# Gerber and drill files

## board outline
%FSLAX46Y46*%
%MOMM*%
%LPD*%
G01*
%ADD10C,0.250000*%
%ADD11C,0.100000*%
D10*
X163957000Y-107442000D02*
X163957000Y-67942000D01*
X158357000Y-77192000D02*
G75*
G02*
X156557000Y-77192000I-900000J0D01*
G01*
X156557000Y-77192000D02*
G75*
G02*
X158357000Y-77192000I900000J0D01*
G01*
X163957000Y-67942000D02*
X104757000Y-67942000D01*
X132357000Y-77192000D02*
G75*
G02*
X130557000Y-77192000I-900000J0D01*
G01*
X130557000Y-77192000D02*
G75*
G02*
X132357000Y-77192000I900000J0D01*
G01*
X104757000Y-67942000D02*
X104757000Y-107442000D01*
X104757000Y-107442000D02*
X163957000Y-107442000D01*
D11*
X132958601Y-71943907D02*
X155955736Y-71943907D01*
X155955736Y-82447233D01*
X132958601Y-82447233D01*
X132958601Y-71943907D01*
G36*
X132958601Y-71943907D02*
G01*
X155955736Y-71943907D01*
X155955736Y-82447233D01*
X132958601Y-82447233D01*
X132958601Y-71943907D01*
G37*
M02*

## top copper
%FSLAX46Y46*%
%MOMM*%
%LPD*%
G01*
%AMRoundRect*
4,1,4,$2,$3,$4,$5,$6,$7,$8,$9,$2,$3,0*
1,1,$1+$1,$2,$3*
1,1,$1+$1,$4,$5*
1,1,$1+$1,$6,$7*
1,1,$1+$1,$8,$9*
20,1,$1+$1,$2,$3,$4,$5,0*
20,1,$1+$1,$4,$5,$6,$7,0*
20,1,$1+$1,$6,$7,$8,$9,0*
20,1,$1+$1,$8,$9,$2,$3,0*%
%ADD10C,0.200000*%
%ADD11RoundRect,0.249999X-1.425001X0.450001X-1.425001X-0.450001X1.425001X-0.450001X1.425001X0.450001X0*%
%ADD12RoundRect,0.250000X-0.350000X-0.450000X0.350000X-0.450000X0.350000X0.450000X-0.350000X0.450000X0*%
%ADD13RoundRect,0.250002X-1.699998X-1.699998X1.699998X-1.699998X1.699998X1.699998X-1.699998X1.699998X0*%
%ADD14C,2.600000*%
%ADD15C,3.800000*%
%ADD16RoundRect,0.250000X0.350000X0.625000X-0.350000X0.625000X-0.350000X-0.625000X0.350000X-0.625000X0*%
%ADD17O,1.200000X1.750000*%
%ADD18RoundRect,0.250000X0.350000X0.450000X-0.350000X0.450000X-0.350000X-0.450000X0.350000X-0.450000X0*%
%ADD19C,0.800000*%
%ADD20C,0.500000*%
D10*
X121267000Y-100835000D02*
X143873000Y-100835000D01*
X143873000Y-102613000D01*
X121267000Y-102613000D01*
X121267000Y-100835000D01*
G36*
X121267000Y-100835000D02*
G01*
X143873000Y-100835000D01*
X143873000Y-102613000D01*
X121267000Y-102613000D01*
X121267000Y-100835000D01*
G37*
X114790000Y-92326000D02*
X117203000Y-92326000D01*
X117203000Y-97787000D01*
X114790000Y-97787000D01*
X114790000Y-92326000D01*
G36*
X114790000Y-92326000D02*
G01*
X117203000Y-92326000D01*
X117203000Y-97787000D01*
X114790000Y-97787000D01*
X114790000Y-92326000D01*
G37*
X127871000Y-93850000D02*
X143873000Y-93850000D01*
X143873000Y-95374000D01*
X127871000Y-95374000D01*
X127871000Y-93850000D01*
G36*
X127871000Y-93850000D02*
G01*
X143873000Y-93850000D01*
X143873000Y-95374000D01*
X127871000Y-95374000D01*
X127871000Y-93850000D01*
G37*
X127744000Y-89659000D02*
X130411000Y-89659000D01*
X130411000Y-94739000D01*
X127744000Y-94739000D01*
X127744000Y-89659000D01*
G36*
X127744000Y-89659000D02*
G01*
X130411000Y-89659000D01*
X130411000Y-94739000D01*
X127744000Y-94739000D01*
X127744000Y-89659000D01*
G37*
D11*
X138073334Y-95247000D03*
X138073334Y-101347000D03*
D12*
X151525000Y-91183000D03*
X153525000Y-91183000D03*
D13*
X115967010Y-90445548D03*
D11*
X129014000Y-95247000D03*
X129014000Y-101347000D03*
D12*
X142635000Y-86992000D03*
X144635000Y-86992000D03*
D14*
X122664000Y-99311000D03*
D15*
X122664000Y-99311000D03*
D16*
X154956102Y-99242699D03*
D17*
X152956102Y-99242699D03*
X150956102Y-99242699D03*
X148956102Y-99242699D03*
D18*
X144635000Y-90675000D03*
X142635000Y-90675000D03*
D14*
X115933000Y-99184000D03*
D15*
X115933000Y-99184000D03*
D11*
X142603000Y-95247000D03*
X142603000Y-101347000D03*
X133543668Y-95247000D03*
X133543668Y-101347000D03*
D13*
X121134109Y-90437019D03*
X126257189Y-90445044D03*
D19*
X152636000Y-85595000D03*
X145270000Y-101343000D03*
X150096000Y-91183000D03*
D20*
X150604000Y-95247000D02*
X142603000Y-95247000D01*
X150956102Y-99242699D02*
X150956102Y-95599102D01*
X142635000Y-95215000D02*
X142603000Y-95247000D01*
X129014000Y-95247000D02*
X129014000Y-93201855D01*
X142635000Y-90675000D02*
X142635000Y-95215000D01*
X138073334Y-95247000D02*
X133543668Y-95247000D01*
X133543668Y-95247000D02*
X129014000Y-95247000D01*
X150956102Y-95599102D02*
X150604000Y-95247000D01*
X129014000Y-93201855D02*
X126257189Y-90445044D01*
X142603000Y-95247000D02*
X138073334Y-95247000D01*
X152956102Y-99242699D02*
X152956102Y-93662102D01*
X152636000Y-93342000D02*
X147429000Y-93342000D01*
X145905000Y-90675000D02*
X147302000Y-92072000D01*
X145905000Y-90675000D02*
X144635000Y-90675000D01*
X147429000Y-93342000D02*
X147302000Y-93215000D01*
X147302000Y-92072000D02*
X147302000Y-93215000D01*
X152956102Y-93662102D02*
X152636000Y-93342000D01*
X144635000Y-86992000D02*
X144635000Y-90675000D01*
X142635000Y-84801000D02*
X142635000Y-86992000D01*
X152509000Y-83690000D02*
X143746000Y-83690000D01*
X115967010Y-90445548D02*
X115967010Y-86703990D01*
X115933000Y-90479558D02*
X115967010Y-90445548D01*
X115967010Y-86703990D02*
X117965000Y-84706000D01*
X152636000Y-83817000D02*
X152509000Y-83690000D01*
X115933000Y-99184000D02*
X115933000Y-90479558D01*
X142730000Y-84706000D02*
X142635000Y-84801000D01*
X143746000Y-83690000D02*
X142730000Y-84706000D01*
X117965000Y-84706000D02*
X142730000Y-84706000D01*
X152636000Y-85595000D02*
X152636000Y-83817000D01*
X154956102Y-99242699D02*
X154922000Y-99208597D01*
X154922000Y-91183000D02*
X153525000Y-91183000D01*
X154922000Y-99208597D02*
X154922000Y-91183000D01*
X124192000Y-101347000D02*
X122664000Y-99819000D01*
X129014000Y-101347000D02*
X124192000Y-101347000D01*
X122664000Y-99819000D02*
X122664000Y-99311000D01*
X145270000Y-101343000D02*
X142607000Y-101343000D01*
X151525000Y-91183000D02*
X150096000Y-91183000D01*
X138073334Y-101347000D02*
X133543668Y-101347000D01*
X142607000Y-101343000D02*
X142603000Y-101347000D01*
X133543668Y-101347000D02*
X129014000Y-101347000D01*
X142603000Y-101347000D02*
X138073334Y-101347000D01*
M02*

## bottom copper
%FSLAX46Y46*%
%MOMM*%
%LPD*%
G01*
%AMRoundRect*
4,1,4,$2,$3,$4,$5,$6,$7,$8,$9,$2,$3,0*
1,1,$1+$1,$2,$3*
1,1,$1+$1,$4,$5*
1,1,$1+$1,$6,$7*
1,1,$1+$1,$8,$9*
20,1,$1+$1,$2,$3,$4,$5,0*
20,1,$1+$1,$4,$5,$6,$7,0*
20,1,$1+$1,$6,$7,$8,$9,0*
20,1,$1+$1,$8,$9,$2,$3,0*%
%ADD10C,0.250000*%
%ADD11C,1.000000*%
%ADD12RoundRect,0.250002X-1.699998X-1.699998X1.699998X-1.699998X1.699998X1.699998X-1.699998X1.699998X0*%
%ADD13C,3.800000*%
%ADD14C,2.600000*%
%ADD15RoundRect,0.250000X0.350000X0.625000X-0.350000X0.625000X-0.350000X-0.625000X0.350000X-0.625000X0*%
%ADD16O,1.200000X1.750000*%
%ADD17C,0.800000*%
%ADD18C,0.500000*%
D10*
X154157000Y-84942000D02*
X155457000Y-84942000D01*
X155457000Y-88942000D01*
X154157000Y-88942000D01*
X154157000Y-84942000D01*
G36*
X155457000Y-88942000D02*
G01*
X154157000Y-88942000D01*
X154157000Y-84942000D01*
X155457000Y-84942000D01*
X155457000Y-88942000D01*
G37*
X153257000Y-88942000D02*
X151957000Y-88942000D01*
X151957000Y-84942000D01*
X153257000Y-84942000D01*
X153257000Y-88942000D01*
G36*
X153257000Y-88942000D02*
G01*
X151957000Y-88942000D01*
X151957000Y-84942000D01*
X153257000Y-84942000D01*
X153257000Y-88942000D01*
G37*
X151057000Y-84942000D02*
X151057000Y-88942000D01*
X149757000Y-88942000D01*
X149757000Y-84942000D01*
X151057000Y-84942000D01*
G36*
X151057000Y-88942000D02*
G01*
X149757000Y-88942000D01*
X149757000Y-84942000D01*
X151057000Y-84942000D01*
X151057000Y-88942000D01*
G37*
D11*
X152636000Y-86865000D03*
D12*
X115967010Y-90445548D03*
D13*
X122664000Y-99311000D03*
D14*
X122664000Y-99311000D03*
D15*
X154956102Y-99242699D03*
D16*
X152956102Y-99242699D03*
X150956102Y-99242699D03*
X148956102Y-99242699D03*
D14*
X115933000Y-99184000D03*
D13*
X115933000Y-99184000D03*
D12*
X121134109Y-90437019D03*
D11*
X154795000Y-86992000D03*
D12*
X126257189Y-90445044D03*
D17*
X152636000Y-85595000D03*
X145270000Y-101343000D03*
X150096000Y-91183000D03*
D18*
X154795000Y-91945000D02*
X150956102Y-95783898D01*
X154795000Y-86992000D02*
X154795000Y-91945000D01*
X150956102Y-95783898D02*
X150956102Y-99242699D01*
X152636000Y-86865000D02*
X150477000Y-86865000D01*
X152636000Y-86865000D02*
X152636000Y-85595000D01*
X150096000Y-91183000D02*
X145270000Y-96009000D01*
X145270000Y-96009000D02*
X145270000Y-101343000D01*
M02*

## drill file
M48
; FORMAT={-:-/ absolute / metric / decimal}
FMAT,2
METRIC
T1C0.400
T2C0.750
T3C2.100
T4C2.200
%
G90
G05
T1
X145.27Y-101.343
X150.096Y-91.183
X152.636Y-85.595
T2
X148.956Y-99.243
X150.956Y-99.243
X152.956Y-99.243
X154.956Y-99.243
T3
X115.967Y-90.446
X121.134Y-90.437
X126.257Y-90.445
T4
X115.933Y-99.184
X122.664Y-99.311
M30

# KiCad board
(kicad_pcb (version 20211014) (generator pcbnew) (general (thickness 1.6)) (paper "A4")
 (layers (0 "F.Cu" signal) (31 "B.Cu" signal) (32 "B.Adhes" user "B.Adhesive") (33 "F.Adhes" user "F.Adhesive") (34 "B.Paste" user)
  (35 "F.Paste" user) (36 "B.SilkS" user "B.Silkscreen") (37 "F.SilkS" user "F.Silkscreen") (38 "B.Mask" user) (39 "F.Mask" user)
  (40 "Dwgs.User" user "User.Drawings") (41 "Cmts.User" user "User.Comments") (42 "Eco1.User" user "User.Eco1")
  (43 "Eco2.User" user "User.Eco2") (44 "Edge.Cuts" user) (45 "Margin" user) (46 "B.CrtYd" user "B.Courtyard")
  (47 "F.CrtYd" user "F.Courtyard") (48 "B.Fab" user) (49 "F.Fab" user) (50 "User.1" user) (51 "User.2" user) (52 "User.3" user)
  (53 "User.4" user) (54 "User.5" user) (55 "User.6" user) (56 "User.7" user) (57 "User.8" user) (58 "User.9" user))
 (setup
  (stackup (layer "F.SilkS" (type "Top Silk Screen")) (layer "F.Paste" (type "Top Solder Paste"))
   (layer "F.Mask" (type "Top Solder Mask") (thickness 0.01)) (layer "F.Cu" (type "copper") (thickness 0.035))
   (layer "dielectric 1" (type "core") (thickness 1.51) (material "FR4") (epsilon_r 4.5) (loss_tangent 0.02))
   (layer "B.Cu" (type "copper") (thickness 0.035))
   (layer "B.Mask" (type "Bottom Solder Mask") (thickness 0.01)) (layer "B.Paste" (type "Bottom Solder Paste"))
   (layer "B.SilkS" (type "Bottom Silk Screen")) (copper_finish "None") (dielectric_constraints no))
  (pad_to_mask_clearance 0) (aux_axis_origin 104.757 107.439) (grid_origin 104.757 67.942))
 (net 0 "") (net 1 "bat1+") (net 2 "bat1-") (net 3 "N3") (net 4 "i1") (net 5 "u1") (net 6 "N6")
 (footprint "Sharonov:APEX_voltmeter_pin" (layer "F.Cu") (at 152.636 86.865)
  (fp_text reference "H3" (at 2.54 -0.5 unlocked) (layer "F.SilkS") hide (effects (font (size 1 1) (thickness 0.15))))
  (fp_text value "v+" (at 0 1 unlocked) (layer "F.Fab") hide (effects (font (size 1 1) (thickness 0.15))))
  (pad "1" smd circle (at 0 0) (size 1 1) (layers "B.Cu") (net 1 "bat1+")))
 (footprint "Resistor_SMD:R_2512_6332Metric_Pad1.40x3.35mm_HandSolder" (layer "F.Cu") (at 138.073334 98.297 -90)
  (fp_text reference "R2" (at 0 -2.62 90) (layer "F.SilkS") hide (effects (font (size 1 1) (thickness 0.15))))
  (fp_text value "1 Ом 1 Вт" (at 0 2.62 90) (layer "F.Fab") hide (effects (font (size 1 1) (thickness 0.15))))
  (pad "1" smd roundrect locked (at -3.05 0 270) (size 1.4 3.35) (layers "F.Cu" "F.Paste" "F.Mask") (roundrect_rratio 0.1785707143)
   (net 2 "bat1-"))
  (pad "2" smd roundrect locked (at 3.05 0 270) (size 1.4 3.35) (layers "F.Cu" "F.Paste" "F.Mask") (roundrect_rratio 0.1785707143)
   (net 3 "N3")))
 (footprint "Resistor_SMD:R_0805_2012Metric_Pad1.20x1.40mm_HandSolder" (layer "F.Cu") (at 152.525 91.183)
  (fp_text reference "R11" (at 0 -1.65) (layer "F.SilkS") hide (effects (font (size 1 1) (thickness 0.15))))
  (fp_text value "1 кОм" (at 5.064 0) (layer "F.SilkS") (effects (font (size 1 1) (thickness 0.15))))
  (pad "1" smd roundrect locked (at -1 0) (size 1.2 1.4) (layers "F.Cu" "F.Paste" "F.Mask") (roundrect_rratio 0.2083333333) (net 3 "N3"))
  (pad "2" smd roundrect locked (at 1 0) (size 1.2 1.4) (layers "F.Cu" "F.Paste" "F.Mask") (roundrect_rratio 0.2083333333) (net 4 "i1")))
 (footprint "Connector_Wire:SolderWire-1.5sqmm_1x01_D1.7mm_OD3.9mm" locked (layer "F.Cu") (at 115.96701 90.445548)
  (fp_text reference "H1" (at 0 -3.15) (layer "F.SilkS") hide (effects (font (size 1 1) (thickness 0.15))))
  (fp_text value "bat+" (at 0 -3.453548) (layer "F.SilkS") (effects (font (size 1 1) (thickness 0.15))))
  (pad "1" thru_hole roundrect locked (at 0 0) (size 3.9 3.9) (drill 2.1) (layers *.Cu *.Mask) (roundrect_rratio 0.06410307692)
   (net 1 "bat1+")))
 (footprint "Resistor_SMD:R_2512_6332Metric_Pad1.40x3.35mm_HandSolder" (layer "F.Cu") (at 129.014 98.297 -90)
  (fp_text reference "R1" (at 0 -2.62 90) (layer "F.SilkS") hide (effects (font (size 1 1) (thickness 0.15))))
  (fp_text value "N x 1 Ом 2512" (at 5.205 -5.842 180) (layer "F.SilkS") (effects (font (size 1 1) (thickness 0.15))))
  (pad "1" smd roundrect locked (at -3.05 0 270) (size 1.4 3.35) (layers "F.Cu" "F.Paste" "F.Mask") (roundrect_rratio 0.1785707143)
   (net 2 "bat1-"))
  (pad "2" smd roundrect locked (at 3.05 0 270) (size 1.4 3.35) (layers "F.Cu" "F.Paste" "F.Mask") (roundrect_rratio 0.1785707143)
   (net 3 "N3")))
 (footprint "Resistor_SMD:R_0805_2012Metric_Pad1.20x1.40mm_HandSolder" (layer "F.Cu") (at 143.635 86.992)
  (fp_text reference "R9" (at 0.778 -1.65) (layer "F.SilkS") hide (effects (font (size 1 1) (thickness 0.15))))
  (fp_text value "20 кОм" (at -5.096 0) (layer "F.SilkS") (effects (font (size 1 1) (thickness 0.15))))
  (pad "1" smd roundrect locked (at -1 0) (size 1.2 1.4) (layers "F.Cu" "F.Paste" "F.Mask") (roundrect_rratio 0.2083333333) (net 1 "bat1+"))
  (pad "2" smd roundrect locked (at 1 0) (size 1.2 1.4) (layers "F.Cu" "F.Paste" "F.Mask") (roundrect_rratio 0.2083333333) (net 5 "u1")))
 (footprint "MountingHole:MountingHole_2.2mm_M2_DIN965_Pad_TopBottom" (layer "F.Cu") (at 122.664 99.311)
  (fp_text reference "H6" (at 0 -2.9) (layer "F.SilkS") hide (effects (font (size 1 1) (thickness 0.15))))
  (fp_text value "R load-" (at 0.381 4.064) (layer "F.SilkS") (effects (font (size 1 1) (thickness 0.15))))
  (pad "1" connect circle locked (at 0 0) (size 3.8 3.8) (layers "B.Cu" "B.Mask") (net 3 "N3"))
  (pad "1" thru_hole circle locked (at 0 0) (size 2.6 2.6) (drill 2.2) (layers *.Cu *.Mask) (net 3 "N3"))
  (pad "1" connect circle locked (at 0 0) (size 3.8 3.8) (layers "F.Cu" "F.Mask") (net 3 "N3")))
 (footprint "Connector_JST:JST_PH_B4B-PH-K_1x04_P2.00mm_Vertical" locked (layer "F.Cu") (at 154.956102 99.242699 180)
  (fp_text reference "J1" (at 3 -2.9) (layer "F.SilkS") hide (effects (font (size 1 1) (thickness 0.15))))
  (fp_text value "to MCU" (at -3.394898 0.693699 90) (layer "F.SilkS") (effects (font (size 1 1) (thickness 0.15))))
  (pad "1" thru_hole roundrect locked (at 0 0 180) (size 1.2 1.75) (drill 0.75) (layers *.Cu *.Mask) (roundrect_rratio 0.2083333333)
   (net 4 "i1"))
  (pad "2" thru_hole oval locked (at 2 0 180) (size 1.2 1.75) (drill 0.75) (layers *.Cu *.Mask) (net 5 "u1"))
  (pad "3" thru_hole oval locked (at 4 0 180) (size 1.2 1.75) (drill 0.75) (layers *.Cu *.Mask) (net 2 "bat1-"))
  (pad "4" thru_hole oval locked (at 6 0 180) (size 1.2 1.75) (drill 0.75) (layers *.Cu *.Mask) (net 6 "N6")))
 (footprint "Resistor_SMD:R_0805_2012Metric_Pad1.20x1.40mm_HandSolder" (layer "F.Cu") (at 143.635 90.675 180)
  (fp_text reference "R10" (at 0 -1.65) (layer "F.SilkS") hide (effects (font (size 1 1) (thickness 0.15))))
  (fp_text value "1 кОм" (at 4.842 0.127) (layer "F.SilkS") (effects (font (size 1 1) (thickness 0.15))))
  (pad "1" smd roundrect locked (at -1 0 180) (size 1.2 1.4) (layers "F.Cu" "F.Paste" "F.Mask") (roundrect_rratio 0.2083333333) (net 5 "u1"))
  (pad "2" smd roundrect locked (at 1 0 180) (size 1.2 1.4) (layers "F.Cu" "F.Paste" "F.Mask") (roundrect_rratio 0.2083333333)
   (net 2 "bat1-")))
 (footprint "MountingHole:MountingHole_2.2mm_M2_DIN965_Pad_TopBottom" (layer "F.Cu") (at 115.933 99.184)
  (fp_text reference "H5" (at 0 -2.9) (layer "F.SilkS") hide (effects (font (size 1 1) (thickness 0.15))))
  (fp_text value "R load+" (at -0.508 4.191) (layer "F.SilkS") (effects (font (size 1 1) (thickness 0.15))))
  (pad "1" thru_hole circle locked (at 0 0) (size 2.6 2.6) (drill 2.2) (layers *.Cu *.Mask) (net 1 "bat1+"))
  (pad "1" connect circle locked (at 0 0) (size 3.8 3.8) (layers "F.Cu" "F.Mask") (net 1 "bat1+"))
  (pad "1" connect circle locked (at 0 0) (size 3.8 3.8) (layers "B.Cu" "B.Mask") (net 1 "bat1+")))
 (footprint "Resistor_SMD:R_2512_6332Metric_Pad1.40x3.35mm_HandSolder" (layer "F.Cu") (at 142.603 98.297 -90)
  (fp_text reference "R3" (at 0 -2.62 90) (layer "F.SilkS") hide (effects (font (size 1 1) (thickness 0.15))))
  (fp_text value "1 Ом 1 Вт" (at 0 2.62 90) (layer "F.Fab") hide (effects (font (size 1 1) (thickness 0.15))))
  (pad "1" smd roundrect locked (at -3.05 0 270) (size 1.4 3.35) (layers "F.Cu" "F.Paste" "F.Mask") (roundrect_rratio 0.1785707143)
   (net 2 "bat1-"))
  (pad "2" smd roundrect locked (at 3.05 0 270) (size 1.4 3.35) (layers "F.Cu" "F.Paste" "F.Mask") (roundrect_rratio 0.1785707143)
   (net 3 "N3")))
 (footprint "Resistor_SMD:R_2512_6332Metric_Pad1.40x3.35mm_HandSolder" (layer "F.Cu") (at 133.543668 98.297 -90)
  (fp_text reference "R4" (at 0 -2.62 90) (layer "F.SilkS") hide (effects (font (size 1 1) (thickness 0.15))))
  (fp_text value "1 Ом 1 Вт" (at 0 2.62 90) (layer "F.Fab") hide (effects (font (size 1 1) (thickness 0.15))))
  (pad "1" smd roundrect locked (at -3.05 0 270) (size 1.4 3.35) (layers "F.Cu" "F.Paste" "F.Mask") (roundrect_rratio 0.1785707143)
   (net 2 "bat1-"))
  (pad "2" smd roundrect locked (at 3.05 0 270) (size 1.4 3.35) (layers "F.Cu" "F.Paste" "F.Mask") (roundrect_rratio 0.1785707143)
   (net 3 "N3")))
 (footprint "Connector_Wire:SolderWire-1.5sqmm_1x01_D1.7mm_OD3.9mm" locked (layer "F.Cu") (at 121.134109 90.437019)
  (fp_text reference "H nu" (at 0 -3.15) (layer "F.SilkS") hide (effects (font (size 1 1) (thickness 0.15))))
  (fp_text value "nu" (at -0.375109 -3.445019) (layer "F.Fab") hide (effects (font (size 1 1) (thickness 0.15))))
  (pad "1" thru_hole roundrect locked (at 0 0) (size 3.9 3.9) (drill 2.1) (layers *.Cu *.Mask) (roundrect_rratio 0.06410307692)))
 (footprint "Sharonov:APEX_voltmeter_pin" (layer "F.Cu") (at 154.795 86.992)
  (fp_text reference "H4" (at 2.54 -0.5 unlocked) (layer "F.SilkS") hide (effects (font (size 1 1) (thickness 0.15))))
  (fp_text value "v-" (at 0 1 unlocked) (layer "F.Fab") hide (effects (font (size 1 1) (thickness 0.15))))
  (pad "1" smd circle (at 0 0) (size 1 1) (layers "B.Cu") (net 2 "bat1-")))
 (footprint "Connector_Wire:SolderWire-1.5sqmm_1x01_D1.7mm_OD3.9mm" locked (layer "F.Cu") (at 126.257189 90.445044)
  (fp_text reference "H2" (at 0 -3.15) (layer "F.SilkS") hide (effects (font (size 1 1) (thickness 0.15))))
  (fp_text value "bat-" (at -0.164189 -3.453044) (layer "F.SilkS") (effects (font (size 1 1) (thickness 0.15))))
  (pad "1" thru_hole roundrect locked (at 0 0) (size 3.9 3.9) (drill 2.1) (layers *.Cu *.Mask) (roundrect_rratio 0.06410307692)
   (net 2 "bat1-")))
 (gr_rect (start 143.873 102.613) (end 121.267 100.835) (layer "F.Cu") (width 0.2) (fill solid))
 (gr_rect (start 114.79 92.326) (end 117.203 97.787) (layer "F.Cu") (width 0.2) (fill solid))
 (gr_rect (start 127.871 95.374) (end 143.873 93.85) (layer "F.Cu") (width 0.2) (fill solid))
 (gr_rect (start 130.411 94.739) (end 127.744 89.659) (layer "F.Cu") (width 0.2) (fill solid))
 (gr_poly locked
  (pts (xy 154.157 84.942) (xy 155.457 84.942) (xy 155.457 88.942) (xy 154.157 88.942)) (layer "B.Cu") (width 0.25) (fill solid))
 (gr_poly locked
  (pts (xy 153.257 88.942) (xy 151.957 88.942) (xy 151.957 84.942) (xy 153.257 84.942)) (layer "B.Cu") (width 0.25) (fill solid))
 (gr_poly locked
  (pts (xy 151.057 84.942) (xy 151.057 88.942) (xy 149.757 88.942) (xy 149.757 84.942)) (layer "B.Cu") (width 0.25) (fill solid))
 (gr_line locked (start 163.957 107.442) (end 163.957 67.942) (layer "Edge.Cuts") (width 0.25))
 (gr_circle locked (center 157.457 77.192) (end 158.357 77.192) (layer "Edge.Cuts") (width 0.25) (fill none))
 (gr_line locked (start 163.957 67.942) (end 104.757 67.942) (layer "Edge.Cuts") (width 0.25))
 (gr_circle locked (center 131.457 77.192) (end 132.357 77.192) (layer "Edge.Cuts") (width 0.25) (fill none))
 (gr_line locked (start 104.757 67.942) (end 104.757 107.442) (layer "Edge.Cuts") (width 0.25))
 (gr_line locked (start 104.757 107.442) (end 163.957 107.442) (layer "Edge.Cuts") (width 0.25))
 (gr_rect locked (start 132.958601 71.943907) (end 155.955736 82.447233) (layer "Edge.Cuts") (width 0.1) (fill solid))
 (segment (start 150.604 95.247) (end 142.603 95.247) (width 0.5) (layer "F.Cu") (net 2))
 (segment (start 150.956102 99.242699) (end 150.956102 95.599102) (width 0.5) (layer "F.Cu") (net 2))
 (segment (start 142.635 95.215) (end 142.603 95.247) (width 0.5) (layer "F.Cu") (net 2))
 (segment (start 129.014 95.247) (end 129.014 93.201855) (width 0.5) (layer "F.Cu") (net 2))
 (segment (start 142.635 90.675) (end 142.635 95.215) (width 0.5) (layer "F.Cu") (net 2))
 (segment (start 138.073334 95.247) (end 133.543668 95.247) (width 0.5) (layer "F.Cu") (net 2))
 (segment (start 133.543668 95.247) (end 129.014 95.247) (width 0.5) (layer "F.Cu") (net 2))
 (segment (start 150.956102 95.599102) (end 150.604 95.247) (width 0.5) (layer "F.Cu") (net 2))
 (segment (start 129.014 93.201855) (end 126.257189 90.445044) (width 0.5) (layer "F.Cu") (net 2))
 (segment (start 142.603 95.247) (end 138.073334 95.247) (width 0.5) (layer "F.Cu") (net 2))
 (segment (start 154.795 91.945) (end 150.956102 95.783898) (width 0.5) (layer "B.Cu") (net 2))
 (segment (start 154.795 86.992) (end 154.795 91.945) (width 0.5) (layer "B.Cu") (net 2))
 (segment (start 150.956102 95.783898) (end 150.956102 99.242699) (width 0.5) (layer "B.Cu") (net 2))
 (segment (start 152.956102 99.242699) (end 152.956102 93.662102) (width 0.5) (layer "F.Cu") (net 5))
 (segment (start 152.636 93.342) (end 147.429 93.342) (width 0.5) (layer "F.Cu") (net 5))
 (segment (start 145.905 90.675) (end 147.302 92.072) (width 0.5) (layer "F.Cu") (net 5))
 (segment (start 145.905 90.675) (end 144.635 90.675) (width 0.5) (layer "F.Cu") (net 5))
 (segment (start 147.429 93.342) (end 147.302 93.215) (width 0.5) (layer "F.Cu") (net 5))
 (segment (start 147.302 92.072) (end 147.302 93.215) (width 0.5) (layer "F.Cu") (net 5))
 (segment (start 152.956102 93.662102) (end 152.636 93.342) (width 0.5) (layer "F.Cu") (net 5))
 (segment (start 144.635 86.992) (end 144.635 90.675) (width 0.5) (layer "F.Cu") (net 5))
 (segment (start 142.635 84.801) (end 142.635 86.992) (width 0.5) (layer "F.Cu") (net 1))
 (segment (start 152.509 83.69) (end 143.746 83.69) (width 0.5) (layer "F.Cu") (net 1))
 (segment (start 115.96701 90.445548) (end 115.96701 86.70399) (width 0.5) (layer "F.Cu") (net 1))
 (segment (start 115.933 90.479558) (end 115.96701 90.445548) (width 0.5) (layer "F.Cu") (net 1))
 (segment (start 115.96701 86.70399) (end 117.965 84.706) (width 0.5) (layer "F.Cu") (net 1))
 (segment (start 152.636 83.817) (end 152.509 83.69) (width 0.5) (layer "F.Cu") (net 1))
 (segment (start 115.933 99.184) (end 115.933 90.479558) (width 0.5) (layer "F.Cu") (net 1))
 (segment (start 142.73 84.706) (end 142.635 84.801) (width 0.5) (layer "F.Cu") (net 1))
 (segment (start 143.746 83.69) (end 142.73 84.706) (width 0.5) (layer "F.Cu") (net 1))
 (segment (start 117.965 84.706) (end 142.73 84.706) (width 0.5) (layer "F.Cu") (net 1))
 (segment (start 152.636 85.595) (end 152.636 83.817) (width 0.5) (layer "F.Cu") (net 1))
 (via (at 152.636 85.595) (size 0.8) (drill 0.4) (layers "F.Cu" "B.Cu") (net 1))
 (segment (start 152.636 86.865) (end 150.477 86.865) (width 0.5) (layer "B.Cu") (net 1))
 (segment (start 152.636 86.865) (end 152.636 85.595) (width 0.5) (layer "B.Cu") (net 1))
 (segment (start 154.956102 99.242699) (end 154.922 99.208597) (width 0.5) (layer "F.Cu") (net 4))
 (segment (start 154.922 91.183) (end 153.525 91.183) (width 0.5) (layer "F.Cu") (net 4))
 (segment (start 154.922 99.208597) (end 154.922 91.183) (width 0.5) (layer "F.Cu") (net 4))
 (segment (start 124.192 101.347) (end 122.664 99.819) (width 0.5) (layer "F.Cu") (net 3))
 (segment (start 129.014 101.347) (end 124.192 101.347) (width 0.5) (layer "F.Cu") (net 3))
 (segment (start 122.664 99.819) (end 122.664 99.311) (width 0.5) (layer "F.Cu") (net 3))
 (segment (start 145.27 101.343) (end 142.607 101.343) (width 0.5) (layer "F.Cu") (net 3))
 (segment (start 151.525 91.183) (end 150.096 91.183) (width 0.5) (layer "F.Cu") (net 3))
 (segment (start 138.073334 101.347) (end 133.543668 101.347) (width 0.5) (layer "F.Cu") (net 3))
 (segment (start 142.607 101.343) (end 142.603 101.347) (width 0.5) (layer "F.Cu") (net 3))
 (segment (start 133.543668 101.347) (end 129.014 101.347) (width 0.5) (layer "F.Cu") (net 3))
 (segment (start 142.603 101.347) (end 138.073334 101.347) (width 0.5) (layer "F.Cu") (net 3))
 (via (at 145.27 101.343) (size 0.8) (drill 0.4) (layers "F.Cu" "B.Cu") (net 3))
 (via (at 150.096 91.183) (size 0.8) (drill 0.4) (layers "F.Cu" "B.Cu") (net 3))
 (segment (start 150.096 91.183) (end 145.27 96.009) (width 0.5) (layer "B.Cu") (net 3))
 (segment (start 145.27 96.009) (end 145.27 101.343) (width 0.5) (layer "B.Cu") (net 3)))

